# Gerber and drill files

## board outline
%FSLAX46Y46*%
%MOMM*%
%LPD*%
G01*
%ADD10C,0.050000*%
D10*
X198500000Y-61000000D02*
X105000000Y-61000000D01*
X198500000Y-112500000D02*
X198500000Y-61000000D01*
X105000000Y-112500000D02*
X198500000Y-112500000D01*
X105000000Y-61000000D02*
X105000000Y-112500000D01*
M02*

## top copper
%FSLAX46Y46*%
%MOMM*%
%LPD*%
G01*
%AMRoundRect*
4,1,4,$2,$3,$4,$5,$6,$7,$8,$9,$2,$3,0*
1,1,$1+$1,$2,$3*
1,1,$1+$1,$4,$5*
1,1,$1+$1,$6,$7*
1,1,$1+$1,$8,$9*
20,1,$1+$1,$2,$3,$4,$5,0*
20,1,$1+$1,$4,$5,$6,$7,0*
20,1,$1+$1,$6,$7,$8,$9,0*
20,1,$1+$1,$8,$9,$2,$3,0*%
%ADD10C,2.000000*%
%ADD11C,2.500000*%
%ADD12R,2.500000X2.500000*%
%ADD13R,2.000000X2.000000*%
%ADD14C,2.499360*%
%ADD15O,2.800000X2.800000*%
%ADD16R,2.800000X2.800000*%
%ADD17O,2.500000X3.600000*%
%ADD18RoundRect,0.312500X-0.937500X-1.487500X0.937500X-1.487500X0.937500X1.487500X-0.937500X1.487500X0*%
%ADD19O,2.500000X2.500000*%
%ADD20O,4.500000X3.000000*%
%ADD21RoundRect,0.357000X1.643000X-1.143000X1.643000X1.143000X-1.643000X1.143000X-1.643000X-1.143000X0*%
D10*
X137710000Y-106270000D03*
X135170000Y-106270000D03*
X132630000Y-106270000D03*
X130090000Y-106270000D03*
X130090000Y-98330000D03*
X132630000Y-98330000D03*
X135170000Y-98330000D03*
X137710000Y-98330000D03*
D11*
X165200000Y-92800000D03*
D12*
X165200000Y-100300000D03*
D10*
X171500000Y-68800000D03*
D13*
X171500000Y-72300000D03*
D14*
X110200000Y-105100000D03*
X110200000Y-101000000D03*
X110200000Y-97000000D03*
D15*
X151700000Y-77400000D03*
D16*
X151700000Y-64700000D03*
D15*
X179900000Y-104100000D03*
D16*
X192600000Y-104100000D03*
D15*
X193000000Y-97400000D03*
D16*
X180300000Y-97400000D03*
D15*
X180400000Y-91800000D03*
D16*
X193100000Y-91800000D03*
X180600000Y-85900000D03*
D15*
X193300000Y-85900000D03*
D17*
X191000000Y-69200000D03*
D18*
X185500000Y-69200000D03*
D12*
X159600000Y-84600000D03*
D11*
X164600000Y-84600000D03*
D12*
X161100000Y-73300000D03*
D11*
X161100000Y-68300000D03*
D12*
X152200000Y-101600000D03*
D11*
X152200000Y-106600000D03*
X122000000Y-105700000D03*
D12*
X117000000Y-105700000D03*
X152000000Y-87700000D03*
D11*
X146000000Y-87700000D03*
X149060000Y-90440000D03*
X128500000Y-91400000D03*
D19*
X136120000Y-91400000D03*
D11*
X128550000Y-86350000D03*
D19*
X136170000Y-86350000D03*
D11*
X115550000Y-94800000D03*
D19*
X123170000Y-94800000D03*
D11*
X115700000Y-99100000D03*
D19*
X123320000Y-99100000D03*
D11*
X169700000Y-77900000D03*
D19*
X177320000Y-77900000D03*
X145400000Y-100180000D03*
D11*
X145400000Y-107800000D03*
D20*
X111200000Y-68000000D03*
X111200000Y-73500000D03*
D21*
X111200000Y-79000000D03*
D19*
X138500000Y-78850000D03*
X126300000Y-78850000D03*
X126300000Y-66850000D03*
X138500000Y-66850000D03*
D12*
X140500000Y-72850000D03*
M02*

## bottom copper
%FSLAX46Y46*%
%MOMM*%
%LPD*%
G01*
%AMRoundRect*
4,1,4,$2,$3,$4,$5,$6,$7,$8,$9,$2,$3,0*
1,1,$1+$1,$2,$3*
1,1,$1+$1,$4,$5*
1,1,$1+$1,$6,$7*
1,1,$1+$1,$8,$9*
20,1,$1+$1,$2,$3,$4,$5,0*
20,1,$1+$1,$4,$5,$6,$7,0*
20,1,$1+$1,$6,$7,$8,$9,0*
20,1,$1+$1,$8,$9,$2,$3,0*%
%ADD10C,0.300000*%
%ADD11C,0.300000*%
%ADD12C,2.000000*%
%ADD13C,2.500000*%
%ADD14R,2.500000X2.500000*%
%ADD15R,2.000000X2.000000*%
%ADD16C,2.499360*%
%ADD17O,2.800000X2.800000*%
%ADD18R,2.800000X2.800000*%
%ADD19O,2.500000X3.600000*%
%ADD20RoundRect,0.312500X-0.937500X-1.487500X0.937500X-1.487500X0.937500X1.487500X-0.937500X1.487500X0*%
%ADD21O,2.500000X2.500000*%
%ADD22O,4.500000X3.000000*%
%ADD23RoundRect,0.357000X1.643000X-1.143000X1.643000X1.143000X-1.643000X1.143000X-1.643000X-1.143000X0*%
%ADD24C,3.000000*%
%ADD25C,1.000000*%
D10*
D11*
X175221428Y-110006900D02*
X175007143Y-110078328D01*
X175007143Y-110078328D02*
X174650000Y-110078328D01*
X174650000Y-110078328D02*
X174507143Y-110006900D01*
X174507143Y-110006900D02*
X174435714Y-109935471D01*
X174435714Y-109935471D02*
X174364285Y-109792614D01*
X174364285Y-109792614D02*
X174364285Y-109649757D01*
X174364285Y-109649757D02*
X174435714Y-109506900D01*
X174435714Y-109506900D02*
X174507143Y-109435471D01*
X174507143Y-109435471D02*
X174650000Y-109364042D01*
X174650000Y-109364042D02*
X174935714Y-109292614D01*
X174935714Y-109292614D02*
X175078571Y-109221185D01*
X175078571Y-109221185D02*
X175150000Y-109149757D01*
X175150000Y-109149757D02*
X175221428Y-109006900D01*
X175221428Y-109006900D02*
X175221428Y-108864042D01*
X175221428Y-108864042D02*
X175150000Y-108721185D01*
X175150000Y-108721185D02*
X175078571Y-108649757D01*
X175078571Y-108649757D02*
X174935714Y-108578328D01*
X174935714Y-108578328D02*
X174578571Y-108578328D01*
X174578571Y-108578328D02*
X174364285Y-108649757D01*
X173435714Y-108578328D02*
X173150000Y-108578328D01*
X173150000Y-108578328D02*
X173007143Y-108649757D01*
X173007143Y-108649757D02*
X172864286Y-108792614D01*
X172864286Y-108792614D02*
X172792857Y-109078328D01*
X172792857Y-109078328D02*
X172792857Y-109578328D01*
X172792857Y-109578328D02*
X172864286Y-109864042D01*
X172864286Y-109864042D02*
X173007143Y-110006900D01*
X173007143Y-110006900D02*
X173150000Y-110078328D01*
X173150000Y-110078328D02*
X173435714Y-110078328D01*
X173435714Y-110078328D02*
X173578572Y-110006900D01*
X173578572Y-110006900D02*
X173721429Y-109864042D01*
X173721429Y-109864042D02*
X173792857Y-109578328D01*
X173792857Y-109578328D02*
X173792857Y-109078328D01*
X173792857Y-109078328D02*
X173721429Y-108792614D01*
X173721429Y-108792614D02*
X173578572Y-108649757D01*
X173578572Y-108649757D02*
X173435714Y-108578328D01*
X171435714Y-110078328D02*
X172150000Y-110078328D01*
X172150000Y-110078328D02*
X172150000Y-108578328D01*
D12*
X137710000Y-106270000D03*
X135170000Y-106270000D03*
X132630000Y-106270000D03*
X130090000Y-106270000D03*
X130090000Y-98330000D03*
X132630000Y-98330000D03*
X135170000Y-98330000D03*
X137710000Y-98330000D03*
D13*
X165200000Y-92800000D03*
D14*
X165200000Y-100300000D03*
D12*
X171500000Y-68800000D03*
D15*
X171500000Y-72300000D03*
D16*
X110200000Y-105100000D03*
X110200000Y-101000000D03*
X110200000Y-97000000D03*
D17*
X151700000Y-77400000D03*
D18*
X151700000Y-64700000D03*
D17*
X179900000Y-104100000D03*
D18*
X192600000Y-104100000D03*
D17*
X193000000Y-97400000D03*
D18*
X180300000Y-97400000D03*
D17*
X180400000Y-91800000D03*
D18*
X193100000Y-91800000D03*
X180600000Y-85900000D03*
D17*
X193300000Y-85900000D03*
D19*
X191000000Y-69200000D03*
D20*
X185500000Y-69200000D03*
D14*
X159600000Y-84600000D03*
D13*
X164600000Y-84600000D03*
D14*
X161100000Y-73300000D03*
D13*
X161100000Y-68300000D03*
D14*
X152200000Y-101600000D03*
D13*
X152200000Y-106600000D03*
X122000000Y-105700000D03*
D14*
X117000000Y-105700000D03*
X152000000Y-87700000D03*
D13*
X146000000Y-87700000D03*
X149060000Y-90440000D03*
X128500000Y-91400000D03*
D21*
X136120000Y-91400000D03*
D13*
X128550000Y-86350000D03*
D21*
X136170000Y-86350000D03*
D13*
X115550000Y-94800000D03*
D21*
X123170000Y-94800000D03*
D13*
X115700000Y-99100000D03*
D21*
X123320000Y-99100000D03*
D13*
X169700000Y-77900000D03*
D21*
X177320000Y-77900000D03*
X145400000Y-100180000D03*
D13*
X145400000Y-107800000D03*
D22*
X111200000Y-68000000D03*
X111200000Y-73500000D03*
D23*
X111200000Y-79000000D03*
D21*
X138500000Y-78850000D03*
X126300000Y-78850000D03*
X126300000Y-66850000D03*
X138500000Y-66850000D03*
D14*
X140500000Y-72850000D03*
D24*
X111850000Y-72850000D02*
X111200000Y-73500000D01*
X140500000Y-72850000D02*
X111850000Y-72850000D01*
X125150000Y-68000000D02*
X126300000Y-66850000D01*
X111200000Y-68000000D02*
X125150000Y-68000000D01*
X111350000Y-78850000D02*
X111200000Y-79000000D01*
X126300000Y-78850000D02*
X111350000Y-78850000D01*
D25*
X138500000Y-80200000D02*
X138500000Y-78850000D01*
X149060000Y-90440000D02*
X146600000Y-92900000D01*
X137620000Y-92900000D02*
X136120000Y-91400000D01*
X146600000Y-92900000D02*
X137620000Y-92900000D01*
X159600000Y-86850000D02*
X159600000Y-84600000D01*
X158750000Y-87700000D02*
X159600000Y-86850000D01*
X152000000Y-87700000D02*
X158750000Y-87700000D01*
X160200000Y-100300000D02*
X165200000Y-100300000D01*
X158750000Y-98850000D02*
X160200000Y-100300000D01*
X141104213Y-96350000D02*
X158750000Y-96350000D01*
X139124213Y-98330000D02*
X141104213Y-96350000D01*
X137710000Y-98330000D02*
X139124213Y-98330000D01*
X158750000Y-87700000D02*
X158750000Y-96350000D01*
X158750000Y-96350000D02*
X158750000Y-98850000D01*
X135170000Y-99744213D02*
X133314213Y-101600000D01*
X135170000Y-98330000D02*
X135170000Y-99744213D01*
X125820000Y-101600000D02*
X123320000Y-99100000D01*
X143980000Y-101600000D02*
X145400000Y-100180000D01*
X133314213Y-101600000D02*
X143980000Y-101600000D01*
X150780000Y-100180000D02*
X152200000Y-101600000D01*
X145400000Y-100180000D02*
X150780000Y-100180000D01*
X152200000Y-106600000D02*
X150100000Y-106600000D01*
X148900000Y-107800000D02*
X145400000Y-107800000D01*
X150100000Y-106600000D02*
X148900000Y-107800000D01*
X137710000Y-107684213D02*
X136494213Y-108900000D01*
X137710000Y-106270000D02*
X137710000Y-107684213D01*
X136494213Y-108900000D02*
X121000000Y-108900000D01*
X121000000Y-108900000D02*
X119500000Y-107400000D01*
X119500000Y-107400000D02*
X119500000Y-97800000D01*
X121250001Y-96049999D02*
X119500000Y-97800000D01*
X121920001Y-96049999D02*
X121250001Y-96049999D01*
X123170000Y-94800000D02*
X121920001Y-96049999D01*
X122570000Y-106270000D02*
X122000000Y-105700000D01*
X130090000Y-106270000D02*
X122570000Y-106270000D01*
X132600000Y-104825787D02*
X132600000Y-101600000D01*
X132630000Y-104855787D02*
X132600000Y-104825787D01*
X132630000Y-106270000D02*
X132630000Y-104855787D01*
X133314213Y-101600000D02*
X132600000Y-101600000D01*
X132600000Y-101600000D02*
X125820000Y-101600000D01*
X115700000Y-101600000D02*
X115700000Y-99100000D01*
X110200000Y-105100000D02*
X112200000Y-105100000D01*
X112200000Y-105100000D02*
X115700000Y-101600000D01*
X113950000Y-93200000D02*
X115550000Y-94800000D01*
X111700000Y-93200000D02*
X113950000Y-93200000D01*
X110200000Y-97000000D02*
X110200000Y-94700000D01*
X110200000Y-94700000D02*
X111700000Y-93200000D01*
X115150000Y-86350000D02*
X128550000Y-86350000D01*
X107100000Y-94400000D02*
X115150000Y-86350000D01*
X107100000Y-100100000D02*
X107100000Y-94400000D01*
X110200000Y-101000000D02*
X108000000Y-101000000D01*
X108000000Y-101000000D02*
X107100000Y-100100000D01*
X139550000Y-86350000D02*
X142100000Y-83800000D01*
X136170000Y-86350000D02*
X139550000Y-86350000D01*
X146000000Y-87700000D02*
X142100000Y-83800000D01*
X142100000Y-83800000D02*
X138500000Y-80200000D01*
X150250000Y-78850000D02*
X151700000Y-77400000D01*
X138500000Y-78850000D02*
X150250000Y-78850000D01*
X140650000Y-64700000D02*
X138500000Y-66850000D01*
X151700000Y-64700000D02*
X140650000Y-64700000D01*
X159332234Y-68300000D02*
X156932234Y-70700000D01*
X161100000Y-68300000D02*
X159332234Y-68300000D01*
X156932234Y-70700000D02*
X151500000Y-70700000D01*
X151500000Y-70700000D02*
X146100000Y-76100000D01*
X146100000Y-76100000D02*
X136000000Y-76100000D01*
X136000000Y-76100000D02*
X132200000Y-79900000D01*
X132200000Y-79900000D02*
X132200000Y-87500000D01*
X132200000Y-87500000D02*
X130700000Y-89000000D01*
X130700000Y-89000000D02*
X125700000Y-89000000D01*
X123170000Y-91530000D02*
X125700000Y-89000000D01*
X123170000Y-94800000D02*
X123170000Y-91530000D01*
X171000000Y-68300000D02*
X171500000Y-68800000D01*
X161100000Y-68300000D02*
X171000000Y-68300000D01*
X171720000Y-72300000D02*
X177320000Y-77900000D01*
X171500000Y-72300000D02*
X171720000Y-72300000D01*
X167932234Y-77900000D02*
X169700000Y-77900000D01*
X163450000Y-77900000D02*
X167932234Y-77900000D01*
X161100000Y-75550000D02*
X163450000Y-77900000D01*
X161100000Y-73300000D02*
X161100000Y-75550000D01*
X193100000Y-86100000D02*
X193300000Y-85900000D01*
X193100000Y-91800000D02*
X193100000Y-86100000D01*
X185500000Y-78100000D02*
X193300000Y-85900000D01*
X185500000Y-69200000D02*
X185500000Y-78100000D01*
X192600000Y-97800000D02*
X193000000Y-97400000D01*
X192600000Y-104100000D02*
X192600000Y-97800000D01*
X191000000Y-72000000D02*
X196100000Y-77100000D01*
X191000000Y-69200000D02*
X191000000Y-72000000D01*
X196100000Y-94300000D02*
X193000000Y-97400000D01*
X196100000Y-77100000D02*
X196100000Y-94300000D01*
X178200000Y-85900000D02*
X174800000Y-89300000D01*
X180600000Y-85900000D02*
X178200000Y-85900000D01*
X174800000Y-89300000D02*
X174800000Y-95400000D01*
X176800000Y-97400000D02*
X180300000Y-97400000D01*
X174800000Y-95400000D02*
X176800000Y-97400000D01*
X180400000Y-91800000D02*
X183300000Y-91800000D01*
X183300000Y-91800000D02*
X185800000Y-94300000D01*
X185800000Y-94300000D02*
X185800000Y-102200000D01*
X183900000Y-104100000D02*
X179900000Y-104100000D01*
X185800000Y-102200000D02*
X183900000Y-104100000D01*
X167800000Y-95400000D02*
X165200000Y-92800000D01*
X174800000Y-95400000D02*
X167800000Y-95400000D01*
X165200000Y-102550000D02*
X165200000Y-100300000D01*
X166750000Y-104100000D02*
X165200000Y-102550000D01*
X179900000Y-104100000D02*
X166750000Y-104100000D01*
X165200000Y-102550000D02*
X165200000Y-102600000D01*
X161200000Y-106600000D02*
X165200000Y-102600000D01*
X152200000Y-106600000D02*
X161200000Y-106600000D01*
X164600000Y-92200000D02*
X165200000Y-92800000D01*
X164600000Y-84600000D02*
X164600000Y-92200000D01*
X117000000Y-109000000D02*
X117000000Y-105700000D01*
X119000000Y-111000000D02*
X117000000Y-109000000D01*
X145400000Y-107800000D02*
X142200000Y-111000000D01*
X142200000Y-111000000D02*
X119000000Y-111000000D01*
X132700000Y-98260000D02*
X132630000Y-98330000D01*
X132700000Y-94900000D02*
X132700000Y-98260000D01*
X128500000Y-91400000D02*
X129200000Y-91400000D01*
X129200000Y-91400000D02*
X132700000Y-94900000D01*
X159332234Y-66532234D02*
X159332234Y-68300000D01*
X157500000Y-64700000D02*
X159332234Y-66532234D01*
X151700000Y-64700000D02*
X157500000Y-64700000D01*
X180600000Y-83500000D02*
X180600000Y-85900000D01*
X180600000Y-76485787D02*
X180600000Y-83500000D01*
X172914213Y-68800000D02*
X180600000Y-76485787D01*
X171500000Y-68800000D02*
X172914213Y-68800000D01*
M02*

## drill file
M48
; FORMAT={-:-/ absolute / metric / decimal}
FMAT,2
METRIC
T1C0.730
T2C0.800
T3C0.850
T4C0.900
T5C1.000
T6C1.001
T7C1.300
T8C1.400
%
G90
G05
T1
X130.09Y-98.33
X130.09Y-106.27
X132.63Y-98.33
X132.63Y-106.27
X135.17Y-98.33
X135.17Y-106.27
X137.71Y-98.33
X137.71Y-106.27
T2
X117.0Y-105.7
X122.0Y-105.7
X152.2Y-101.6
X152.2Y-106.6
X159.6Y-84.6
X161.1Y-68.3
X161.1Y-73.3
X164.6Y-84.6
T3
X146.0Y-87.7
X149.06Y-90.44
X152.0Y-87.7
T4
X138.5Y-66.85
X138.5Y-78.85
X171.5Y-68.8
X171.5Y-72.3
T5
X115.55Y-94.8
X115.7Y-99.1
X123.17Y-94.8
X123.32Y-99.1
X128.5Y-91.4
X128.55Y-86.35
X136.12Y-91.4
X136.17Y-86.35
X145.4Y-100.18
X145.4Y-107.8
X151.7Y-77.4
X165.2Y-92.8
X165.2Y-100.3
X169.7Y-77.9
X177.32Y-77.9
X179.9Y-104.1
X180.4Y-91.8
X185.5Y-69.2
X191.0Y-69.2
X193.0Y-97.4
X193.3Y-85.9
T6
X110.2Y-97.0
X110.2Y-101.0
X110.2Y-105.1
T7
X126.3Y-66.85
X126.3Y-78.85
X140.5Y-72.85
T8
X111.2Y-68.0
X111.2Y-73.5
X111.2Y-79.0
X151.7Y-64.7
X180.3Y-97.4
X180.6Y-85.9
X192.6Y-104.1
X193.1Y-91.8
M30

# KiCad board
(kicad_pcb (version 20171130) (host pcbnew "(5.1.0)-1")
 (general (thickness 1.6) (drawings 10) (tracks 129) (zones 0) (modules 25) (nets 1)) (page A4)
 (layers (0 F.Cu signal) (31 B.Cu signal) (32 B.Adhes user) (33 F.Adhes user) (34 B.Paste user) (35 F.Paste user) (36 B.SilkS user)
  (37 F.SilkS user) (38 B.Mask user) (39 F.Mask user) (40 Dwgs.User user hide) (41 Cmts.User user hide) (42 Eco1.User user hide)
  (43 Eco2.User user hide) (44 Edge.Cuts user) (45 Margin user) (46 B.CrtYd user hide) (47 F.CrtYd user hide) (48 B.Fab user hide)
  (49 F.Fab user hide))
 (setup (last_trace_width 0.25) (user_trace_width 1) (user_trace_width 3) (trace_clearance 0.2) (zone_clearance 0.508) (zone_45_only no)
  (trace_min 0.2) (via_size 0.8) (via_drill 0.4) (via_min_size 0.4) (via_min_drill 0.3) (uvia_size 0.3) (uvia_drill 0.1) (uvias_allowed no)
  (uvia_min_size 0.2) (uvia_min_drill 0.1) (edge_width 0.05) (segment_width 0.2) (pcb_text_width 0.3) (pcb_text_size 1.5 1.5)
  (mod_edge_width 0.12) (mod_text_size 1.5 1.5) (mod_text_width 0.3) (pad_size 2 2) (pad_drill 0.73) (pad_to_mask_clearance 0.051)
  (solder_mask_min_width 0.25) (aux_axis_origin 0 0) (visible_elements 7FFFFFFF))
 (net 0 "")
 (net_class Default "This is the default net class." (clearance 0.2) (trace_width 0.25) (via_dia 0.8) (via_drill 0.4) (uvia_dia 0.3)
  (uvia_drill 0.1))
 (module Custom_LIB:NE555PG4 (layer F.Cu) (at 133.9 102.3 270)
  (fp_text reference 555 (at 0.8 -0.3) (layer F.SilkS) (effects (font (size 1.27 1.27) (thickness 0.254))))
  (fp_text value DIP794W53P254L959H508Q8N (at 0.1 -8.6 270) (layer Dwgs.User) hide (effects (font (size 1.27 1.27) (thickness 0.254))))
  (pad 8 thru_hole circle (at 3.97 -3.81 270) (size 2 2) (drill 0.73) (layers *.Cu *.Mask))
  (pad 7 thru_hole circle (at 3.97 -1.27 270) (size 2 2) (drill 0.73) (layers *.Cu *.Mask))
  (pad 6 thru_hole circle (at 3.97 1.27 270) (size 2 2) (drill 0.73) (layers *.Cu *.Mask))
  (pad 5 thru_hole circle (at 3.97 3.81 270) (size 2 2) (drill 0.73) (layers *.Cu *.Mask))
  (pad 4 thru_hole circle (at -3.97 3.81 270) (size 2 2) (drill 0.73) (layers *.Cu *.Mask))
  (pad 3 thru_hole circle (at -3.97 1.27 270) (size 2 2) (drill 0.73) (layers *.Cu *.Mask))
  (pad 2 thru_hole circle (at -3.97 -1.27 270) (size 2 2) (drill 0.73) (layers *.Cu *.Mask))
  (pad 1 thru_hole circle (at -3.97 -3.81 270) (size 2 2) (drill 0.73) (layers *.Cu *.Mask)))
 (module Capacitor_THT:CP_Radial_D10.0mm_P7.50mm (layer F.Cu) (at 165.2 100.3 90)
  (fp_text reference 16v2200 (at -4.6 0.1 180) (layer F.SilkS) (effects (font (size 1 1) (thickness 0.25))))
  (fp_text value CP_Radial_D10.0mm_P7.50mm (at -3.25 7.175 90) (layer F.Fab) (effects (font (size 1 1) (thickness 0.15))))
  (pad 2 thru_hole circle (at 7.5 0 90) (size 2.5 2.5) (drill 1) (layers *.Cu *.Mask))
  (pad 1 thru_hole rect (at 0 0 90) (size 2.5 2.5) (drill 1) (layers *.Cu *.Mask)))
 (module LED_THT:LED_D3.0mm (layer F.Cu) (at 171.5 71.8 90)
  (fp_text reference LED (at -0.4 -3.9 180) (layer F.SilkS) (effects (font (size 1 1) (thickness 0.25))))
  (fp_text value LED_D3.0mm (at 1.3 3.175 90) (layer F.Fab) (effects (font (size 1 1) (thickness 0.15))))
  (pad 2 thru_hole circle (at 3 0 180) (size 2 2) (drill 0.9) (layers *.Cu *.Mask))
  (pad 1 thru_hole rect (at -0.5 0 90) (size 2 2) (drill 0.9) (layers *.Cu *.Mask)))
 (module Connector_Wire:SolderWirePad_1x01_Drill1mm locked (layer F.Cu) (at 110.2 105.1)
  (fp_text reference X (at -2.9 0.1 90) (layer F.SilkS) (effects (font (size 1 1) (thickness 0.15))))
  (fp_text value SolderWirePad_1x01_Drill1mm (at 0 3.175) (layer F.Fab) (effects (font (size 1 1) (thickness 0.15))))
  (pad 1 thru_hole circle (at 0 0) (size 2.49936 2.49936) (drill 1.00076) (layers *.Cu *.Mask)))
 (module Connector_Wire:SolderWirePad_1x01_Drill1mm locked (layer F.Cu) (at 110.2 101)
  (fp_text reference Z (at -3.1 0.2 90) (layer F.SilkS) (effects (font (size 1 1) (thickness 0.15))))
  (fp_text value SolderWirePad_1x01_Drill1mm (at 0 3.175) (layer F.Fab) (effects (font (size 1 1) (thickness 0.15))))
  (pad 1 thru_hole circle (at 0 0) (size 2.49936 2.49936) (drill 1.00076) (layers *.Cu *.Mask)))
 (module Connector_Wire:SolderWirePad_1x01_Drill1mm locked (layer F.Cu) (at 110.5 97)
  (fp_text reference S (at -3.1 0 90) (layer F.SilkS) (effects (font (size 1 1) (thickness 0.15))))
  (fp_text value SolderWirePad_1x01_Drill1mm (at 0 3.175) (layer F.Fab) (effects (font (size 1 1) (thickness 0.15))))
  (pad 1 thru_hole circle (at -0.3 0) (size 2.49936 2.49936) (drill 1.00076) (layers *.Cu *.Mask)))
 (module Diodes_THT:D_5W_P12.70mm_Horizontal (layer F.Cu) (at 151.7 64.7 270)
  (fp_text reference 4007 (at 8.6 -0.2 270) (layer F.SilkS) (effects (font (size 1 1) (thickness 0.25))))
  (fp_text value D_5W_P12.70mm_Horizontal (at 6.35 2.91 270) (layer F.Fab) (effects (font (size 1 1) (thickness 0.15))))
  (pad 2 thru_hole oval (at 12.7 0 270) (size 2.8 2.8) (drill 1) (layers *.Cu *.Mask))
  (pad 1 thru_hole rect (at 0 0 270) (size 2.8 2.8) (drill 1.4) (layers *.Cu *.Mask)))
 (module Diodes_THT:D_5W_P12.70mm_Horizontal (layer F.Cu) (at 192.6 104.1 180)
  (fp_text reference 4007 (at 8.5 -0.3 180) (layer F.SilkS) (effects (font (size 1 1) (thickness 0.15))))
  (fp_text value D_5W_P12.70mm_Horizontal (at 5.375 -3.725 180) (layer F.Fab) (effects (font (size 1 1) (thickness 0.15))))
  (pad 2 thru_hole oval (at 12.7 0 180) (size 2.8 2.8) (drill 1) (layers *.Cu *.Mask))
  (pad 1 thru_hole rect (at 0 0 180) (size 2.8 2.8) (drill 1.4) (layers *.Cu *.Mask)))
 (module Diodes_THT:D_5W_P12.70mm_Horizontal (layer F.Cu) (at 180.3 97.4)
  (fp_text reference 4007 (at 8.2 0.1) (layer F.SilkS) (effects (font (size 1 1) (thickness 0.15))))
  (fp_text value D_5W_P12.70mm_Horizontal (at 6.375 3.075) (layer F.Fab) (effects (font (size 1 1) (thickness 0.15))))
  (pad 2 thru_hole oval (at 12.7 0) (size 2.8 2.8) (drill 1) (layers *.Cu *.Mask))
  (pad 1 thru_hole rect (at 0 0) (size 2.8 2.8) (drill 1.4) (layers *.Cu *.Mask)))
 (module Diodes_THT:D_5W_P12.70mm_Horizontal (layer F.Cu) (at 193.1 91.8 180)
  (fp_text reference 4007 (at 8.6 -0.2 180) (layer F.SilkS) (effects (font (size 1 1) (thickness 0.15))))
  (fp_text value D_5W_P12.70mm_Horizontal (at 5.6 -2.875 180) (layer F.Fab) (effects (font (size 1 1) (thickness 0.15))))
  (pad 2 thru_hole oval (at 12.7 0 180) (size 2.8 2.8) (drill 1) (layers *.Cu *.Mask))
  (pad 1 thru_hole rect (at 0 0 180) (size 2.8 2.8) (drill 1.4) (layers *.Cu *.Mask)))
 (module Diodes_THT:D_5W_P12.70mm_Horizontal (layer F.Cu) (at 180.6 85.9)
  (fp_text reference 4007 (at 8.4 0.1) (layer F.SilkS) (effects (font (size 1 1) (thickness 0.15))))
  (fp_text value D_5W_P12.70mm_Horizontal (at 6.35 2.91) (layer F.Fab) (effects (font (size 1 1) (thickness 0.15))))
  (pad 1 thru_hole rect (at 0 0) (size 2.8 2.8) (drill 1.4) (layers *.Cu *.Mask))
  (pad 2 thru_hole oval (at 12.7 0) (size 2.8 2.8) (drill 1) (layers *.Cu *.Mask)))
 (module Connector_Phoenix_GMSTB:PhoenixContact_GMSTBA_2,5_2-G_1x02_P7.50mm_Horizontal (layer F.Cu) (at 184.5 66.2)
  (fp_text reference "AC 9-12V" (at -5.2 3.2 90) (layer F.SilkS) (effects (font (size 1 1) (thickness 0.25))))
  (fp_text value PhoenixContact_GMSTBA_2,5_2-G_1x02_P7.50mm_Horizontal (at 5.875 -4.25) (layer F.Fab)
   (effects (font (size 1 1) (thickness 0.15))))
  (pad 2 thru_hole oval (at 6.5 3) (size 2.5 3.6) (drill 1) (layers *.Cu *.Mask))
  (pad 1 thru_hole roundrect (at 1 3) (size 2.5 3.6) (drill 1) (layers *.Cu *.Mask) (roundrect_rratio 0.125)))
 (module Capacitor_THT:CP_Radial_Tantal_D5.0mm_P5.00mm (layer F.Cu) (at 159.6 84.6)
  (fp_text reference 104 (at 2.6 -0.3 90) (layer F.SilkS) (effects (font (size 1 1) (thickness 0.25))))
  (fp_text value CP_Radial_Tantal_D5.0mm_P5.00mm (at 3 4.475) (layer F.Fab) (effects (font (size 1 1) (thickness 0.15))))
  (pad 1 thru_hole rect (at 0 0) (size 2.5 2.5) (drill 0.8) (layers *.Cu *.Mask))
  (pad 2 thru_hole circle (at 5 0) (size 2.5 2.5) (drill 0.8) (layers *.Cu *.Mask)))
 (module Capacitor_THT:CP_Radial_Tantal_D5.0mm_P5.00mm (layer F.Cu) (at 161.1 73.3 90)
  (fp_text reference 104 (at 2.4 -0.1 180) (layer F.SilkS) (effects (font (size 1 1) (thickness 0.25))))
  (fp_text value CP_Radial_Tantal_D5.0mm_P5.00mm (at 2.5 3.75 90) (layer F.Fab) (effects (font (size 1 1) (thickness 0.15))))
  (pad 1 thru_hole rect (at 0 0 90) (size 2.5 2.5) (drill 0.8) (layers *.Cu *.Mask))
  (pad 2 thru_hole circle (at 5 0 90) (size 2.5 2.5) (drill 0.8) (layers *.Cu *.Mask)))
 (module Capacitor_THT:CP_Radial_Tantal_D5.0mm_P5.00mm (layer F.Cu) (at 152.2 101.6 270)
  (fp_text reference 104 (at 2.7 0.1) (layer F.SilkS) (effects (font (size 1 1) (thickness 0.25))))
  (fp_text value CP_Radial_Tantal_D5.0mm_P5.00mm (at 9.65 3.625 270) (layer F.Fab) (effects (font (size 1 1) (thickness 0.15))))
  (pad 1 thru_hole rect (at 0 0 270) (size 2.5 2.5) (drill 0.8) (layers *.Cu *.Mask))
  (pad 2 thru_hole circle (at 5 0 270) (size 2.5 2.5) (drill 0.8) (layers *.Cu *.Mask)))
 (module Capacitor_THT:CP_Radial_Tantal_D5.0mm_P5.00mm (layer F.Cu) (at 117 105.7)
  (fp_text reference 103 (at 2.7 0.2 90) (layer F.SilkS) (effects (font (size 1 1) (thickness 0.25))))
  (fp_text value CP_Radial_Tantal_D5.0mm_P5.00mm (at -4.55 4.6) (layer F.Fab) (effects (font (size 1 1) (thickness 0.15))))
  (pad 2 thru_hole circle (at 5 0) (size 2.5 2.5) (drill 0.8) (layers *.Cu *.Mask))
  (pad 1 thru_hole rect (at 0 0) (size 2.5 2.5) (drill 0.8) (layers *.Cu *.Mask)))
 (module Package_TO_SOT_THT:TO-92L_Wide (layer F.Cu) (at 151.6 87.9 180)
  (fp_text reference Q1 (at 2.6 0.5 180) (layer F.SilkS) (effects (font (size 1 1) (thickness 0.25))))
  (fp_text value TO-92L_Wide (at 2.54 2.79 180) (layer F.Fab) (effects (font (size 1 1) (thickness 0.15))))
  (pad 1 thru_hole rect (at -0.4 0.2 270) (size 2.5 2.5) (drill 0.85) (layers *.Cu *.Mask))
  (pad 3 thru_hole circle (at 5.6 0.2 270) (size 2.5 2.5) (drill 0.85) (layers *.Cu *.Mask))
  (pad 2 thru_hole circle (at 2.54 -2.54 270) (size 2.5 2.5) (drill 0.85) (layers *.Cu *.Mask)))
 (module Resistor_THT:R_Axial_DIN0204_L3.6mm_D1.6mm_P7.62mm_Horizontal (layer F.Cu) (at 128.5 91.4)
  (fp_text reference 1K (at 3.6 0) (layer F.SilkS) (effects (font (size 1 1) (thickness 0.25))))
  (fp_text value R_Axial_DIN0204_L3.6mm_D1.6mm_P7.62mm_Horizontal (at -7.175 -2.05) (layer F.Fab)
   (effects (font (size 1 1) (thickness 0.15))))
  (pad 1 thru_hole circle (at 0 0) (size 2.5 2.5) (drill 1) (layers *.Cu *.Mask))
  (pad 2 thru_hole oval (at 7.62 0 90) (size 2.5 2.5) (drill 1) (layers *.Cu *.Mask)))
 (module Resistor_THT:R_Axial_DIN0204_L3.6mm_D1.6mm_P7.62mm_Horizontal (layer F.Cu) (at 128.55 86.35)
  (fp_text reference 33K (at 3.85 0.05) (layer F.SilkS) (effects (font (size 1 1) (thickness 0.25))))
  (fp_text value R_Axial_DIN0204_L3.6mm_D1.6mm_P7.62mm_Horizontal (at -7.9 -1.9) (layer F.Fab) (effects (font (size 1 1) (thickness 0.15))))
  (pad 1 thru_hole circle (at 0 0) (size 2.5 2.5) (drill 1) (layers *.Cu *.Mask))
  (pad 2 thru_hole oval (at 7.62 0 90) (size 2.5 2.5) (drill 1) (layers *.Cu *.Mask)))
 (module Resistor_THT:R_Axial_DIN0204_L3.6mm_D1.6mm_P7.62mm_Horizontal (layer F.Cu) (at 115.55 94.8)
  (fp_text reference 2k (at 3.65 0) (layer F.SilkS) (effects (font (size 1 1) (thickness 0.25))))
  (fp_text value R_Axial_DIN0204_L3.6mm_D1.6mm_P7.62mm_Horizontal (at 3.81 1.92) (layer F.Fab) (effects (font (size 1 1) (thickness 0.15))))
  (pad 1 thru_hole circle (at 0 0) (size 2.5 2.5) (drill 1) (layers *.Cu *.Mask))
  (pad 2 thru_hole oval (at 7.62 0 90) (size 2.5 2.5) (drill 1) (layers *.Cu *.Mask)))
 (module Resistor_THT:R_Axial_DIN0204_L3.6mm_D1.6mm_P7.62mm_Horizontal (layer F.Cu) (at 115.7 99.1)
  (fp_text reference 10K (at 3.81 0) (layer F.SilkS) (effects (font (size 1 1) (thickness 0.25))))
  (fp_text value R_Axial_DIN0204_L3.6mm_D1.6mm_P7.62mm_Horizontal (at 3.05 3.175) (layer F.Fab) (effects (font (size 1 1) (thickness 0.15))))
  (pad 1 thru_hole circle (at 0 0) (size 2.5 2.5) (drill 1) (layers *.Cu *.Mask))
  (pad 2 thru_hole oval (at 7.62 0 90) (size 2.5 2.5) (drill 1) (layers *.Cu *.Mask)))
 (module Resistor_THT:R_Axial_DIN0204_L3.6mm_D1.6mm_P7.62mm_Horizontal (layer F.Cu) (at 169.7 77.9)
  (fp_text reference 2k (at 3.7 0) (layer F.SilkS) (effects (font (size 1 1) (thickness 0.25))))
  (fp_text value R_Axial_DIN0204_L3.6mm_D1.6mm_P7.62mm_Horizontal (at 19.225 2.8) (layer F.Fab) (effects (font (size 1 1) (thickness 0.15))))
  (pad 1 thru_hole circle (at 0 0) (size 2.5 2.5) (drill 1) (layers *.Cu *.Mask))
  (pad 2 thru_hole oval (at 7.62 0 90) (size 2.5 2.5) (drill 1) (layers *.Cu *.Mask)))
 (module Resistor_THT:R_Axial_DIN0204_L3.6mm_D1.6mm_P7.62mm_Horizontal (layer F.Cu) (at 145.4 107.8 90)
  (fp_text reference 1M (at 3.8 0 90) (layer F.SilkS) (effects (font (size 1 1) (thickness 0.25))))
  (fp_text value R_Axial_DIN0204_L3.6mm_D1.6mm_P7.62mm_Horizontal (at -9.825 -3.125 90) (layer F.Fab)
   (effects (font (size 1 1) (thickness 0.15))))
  (pad 2 thru_hole oval (at 7.62 0 180) (size 2.5 2.5) (drill 1) (layers *.Cu *.Mask))
  (pad 1 thru_hole circle (at 0 0 90) (size 2.5 2.5) (drill 1) (layers *.Cu *.Mask)))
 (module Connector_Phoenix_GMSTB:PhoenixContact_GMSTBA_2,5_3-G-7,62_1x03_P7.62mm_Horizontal (layer F.Cu) (at 108.5 81 90)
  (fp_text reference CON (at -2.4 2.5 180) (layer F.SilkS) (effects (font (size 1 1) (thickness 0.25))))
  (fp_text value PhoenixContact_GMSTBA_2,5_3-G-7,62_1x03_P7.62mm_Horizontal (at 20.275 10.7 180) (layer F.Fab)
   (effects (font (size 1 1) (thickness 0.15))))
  (pad 3 thru_hole oval (at 13 2.7 90) (size 3 4.5) (drill 1.4) (layers *.Cu *.Mask))
  (pad 2 thru_hole oval (at 7.5 2.7 90) (size 3 4.5) (drill 1.4) (layers *.Cu *.Mask))
  (pad 1 thru_hole roundrect (at 2 2.7 90) (size 3 4) (drill 1.4) (layers *.Cu *.Mask) (roundrect_rratio 0.119)))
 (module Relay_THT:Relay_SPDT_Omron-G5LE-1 (layer F.Cu) (at 140.5 72.85 270)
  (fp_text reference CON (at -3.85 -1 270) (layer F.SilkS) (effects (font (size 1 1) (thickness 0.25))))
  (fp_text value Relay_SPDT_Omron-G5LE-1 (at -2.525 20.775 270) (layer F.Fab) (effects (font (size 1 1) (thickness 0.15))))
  (pad 5 thru_hole oval (at 6 2 270) (size 2.5 2.5) (drill 0.9) (layers *.Cu *.Mask))
  (pad 4 thru_hole oval (at 6 14.2 270) (size 2.5 2.5) (drill 1.3) (layers *.Cu *.Mask))
  (pad 3 thru_hole oval (at -6 14.2 270) (size 2.5 2.5) (drill 1.3) (layers *.Cu *.Mask))
  (pad 2 thru_hole oval (at -6 2 270) (size 2.5 2.5) (drill 0.9) (layers *.Cu *.Mask))
  (pad 1 thru_hole rect (at 0 0 270) (size 2.5 2.5) (drill 1.3) (layers *.Cu *.Mask)))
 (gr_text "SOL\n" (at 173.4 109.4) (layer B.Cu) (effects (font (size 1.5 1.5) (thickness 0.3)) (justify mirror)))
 (gr_line (start 198.5 61) (end 105 61) (layer Edge.Cuts) (width 0.05))
 (gr_line (start 198.5 112.5) (end 198.5 61) (layer Edge.Cuts) (width 0.05))
 (gr_line (start 105 112.5) (end 198.5 112.5) (layer Edge.Cuts) (width 0.05))
 (gr_line (start 105 61) (end 105 112.5) (layer Edge.Cuts) (width 0.05))
 (segment (start 111.85 72.85) (end 111.2 73.5) (width 3) (layer B.Cu) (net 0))
 (segment (start 140.5 72.85) (end 111.85 72.85) (width 3) (layer B.Cu) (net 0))
 (segment (start 125.15 68) (end 126.3 66.85) (width 3) (layer B.Cu) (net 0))
 (segment (start 111.2 68) (end 125.15 68) (width 3) (layer B.Cu) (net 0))
 (segment (start 111.35 78.85) (end 111.2 79) (width 3) (layer B.Cu) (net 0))
 (segment (start 126.3 78.85) (end 111.35 78.85) (width 3) (layer B.Cu) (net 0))
 (segment (start 138.5 80.2) (end 138.5 78.85) (width 1) (layer B.Cu) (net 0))
 (segment (start 149.06 90.44) (end 146.6 92.9) (width 1) (layer B.Cu) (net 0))
 (segment (start 137.62 92.9) (end 136.12 91.4) (width 1) (layer B.Cu) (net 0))
 (segment (start 146.6 92.9) (end 137.62 92.9) (width 1) (layer B.Cu) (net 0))
 (segment (start 159.6 86.85) (end 159.6 84.6) (width 1) (layer B.Cu) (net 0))
 (segment (start 158.75 87.7) (end 159.6 86.85) (width 1) (layer B.Cu) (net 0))
 (segment (start 152 87.7) (end 158.75 87.7) (width 1) (layer B.Cu) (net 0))
 (segment (start 160.2 100.3) (end 165.2 100.3) (width 1) (layer B.Cu) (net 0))
 (segment (start 158.75 98.85) (end 160.2 100.3) (width 1) (layer B.Cu) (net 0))
 (segment (start 141.104213 96.35) (end 158.75 96.35) (width 1) (layer B.Cu) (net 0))
 (segment (start 139.124213 98.33) (end 141.104213 96.35) (width 1) (layer B.Cu) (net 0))
 (segment (start 137.71 98.33) (end 139.124213 98.33) (width 1) (layer B.Cu) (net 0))
 (segment (start 158.75 87.7) (end 158.75 96.35) (width 1) (layer B.Cu) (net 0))
 (segment (start 158.75 96.35) (end 158.75 98.85) (width 1) (layer B.Cu) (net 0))
 (segment (start 135.17 99.744213) (end 133.314213 101.6) (width 1) (layer B.Cu) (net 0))
 (segment (start 135.17 98.33) (end 135.17 99.744213) (width 1) (layer B.Cu) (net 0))
 (segment (start 125.82 101.6) (end 123.32 99.1) (width 1) (layer B.Cu) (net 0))
 (segment (start 143.98 101.6) (end 145.4 100.18) (width 1) (layer B.Cu) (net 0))
 (segment (start 133.314213 101.6) (end 143.98 101.6) (width 1) (layer B.Cu) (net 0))
 (segment (start 150.78 100.18) (end 152.2 101.6) (width 1) (layer B.Cu) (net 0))
 (segment (start 145.4 100.18) (end 150.78 100.18) (width 1) (layer B.Cu) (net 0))
 (segment (start 152.2 106.6) (end 150.1 106.6) (width 1) (layer B.Cu) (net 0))
 (segment (start 148.9 107.8) (end 145.4 107.8) (width 1) (layer B.Cu) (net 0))
 (segment (start 150.1 106.6) (end 148.9 107.8) (width 1) (layer B.Cu) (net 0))
 (segment (start 137.71 107.684213) (end 136.494213 108.9) (width 1) (layer B.Cu) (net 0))
 (segment (start 137.71 106.27) (end 137.71 107.684213) (width 1) (layer B.Cu) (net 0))
 (segment (start 136.494213 108.9) (end 121 108.9) (width 1) (layer B.Cu) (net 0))
 (segment (start 121 108.9) (end 119.5 107.4) (width 1) (layer B.Cu) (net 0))
 (segment (start 119.5 107.4) (end 119.5 97.8) (width 1) (layer B.Cu) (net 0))
 (segment (start 121.250001 96.049999) (end 119.5 97.8) (width 1) (layer B.Cu) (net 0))
 (segment (start 121.920001 96.049999) (end 121.250001 96.049999) (width 1) (layer B.Cu) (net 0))
 (segment (start 123.17 94.8) (end 121.920001 96.049999) (width 1) (layer B.Cu) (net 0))
 (segment (start 122.57 106.27) (end 122 105.7) (width 1) (layer B.Cu) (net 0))
 (segment (start 130.09 106.27) (end 122.57 106.27) (width 1) (layer B.Cu) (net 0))
 (segment (start 132.6 104.825787) (end 132.6 101.6) (width 1) (layer B.Cu) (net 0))
 (segment (start 132.63 104.855787) (end 132.6 104.825787) (width 1) (layer B.Cu) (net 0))
 (segment (start 132.63 106.27) (end 132.63 104.855787) (width 1) (layer B.Cu) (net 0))
 (segment (start 133.314213 101.6) (end 132.6 101.6) (width 1) (layer B.Cu) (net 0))
 (segment (start 132.6 101.6) (end 125.82 101.6) (width 1) (layer B.Cu) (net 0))
 (segment (start 115.7 101.6) (end 115.7 99.1) (width 1) (layer B.Cu) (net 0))
 (segment (start 110.2 105.1) (end 112.2 105.1) (width 1) (layer B.Cu) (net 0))
 (segment (start 112.2 105.1) (end 115.7 101.6) (width 1) (layer B.Cu) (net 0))
 (segment (start 113.95 93.2) (end 115.55 94.8) (width 1) (layer B.Cu) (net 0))
 (segment (start 111.7 93.2) (end 113.95 93.2) (width 1) (layer B.Cu) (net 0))
 (segment (start 110.2 97) (end 110.2 94.7) (width 1) (layer B.Cu) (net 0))
 (segment (start 110.2 94.7) (end 111.7 93.2) (width 1) (layer B.Cu) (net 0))
 (segment (start 115.15 86.35) (end 128.55 86.35) (width 1) (layer B.Cu) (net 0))
 (segment (start 107.1 94.4) (end 115.15 86.35) (width 1) (layer B.Cu) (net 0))
 (segment (start 107.1 100.1) (end 107.1 94.4) (width 1) (layer B.Cu) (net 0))
 (segment (start 110.2 101) (end 108 101) (width 1) (layer B.Cu) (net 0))
 (segment (start 108 101) (end 107.1 100.1) (width 1) (layer B.Cu) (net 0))
 (segment (start 139.55 86.35) (end 142.1 83.8) (width 1) (layer B.Cu) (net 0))
 (segment (start 136.17 86.35) (end 139.55 86.35) (width 1) (layer B.Cu) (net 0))
 (segment (start 146 87.7) (end 142.1 83.8) (width 1) (layer B.Cu) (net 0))
 (segment (start 142.1 83.8) (end 138.5 80.2) (width 1) (layer B.Cu) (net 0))
 (segment (start 150.25 78.85) (end 151.7 77.4) (width 1) (layer B.Cu) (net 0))
 (segment (start 138.5 78.85) (end 150.25 78.85) (width 1) (layer B.Cu) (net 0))
 (segment (start 140.65 64.7) (end 138.5 66.85) (width 1) (layer B.Cu) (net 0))
 (segment (start 151.7 64.7) (end 140.65 64.7) (width 1) (layer B.Cu) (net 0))
 (segment (start 159.332234 68.3) (end 156.932234 70.7) (width 1) (layer B.Cu) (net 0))
 (segment (start 161.1 68.3) (end 159.332234 68.3) (width 1) (layer B.Cu) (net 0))
 (segment (start 156.932234 70.7) (end 151.5 70.7) (width 1) (layer B.Cu) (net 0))
 (segment (start 151.5 70.7) (end 146.1 76.1) (width 1) (layer B.Cu) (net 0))
 (segment (start 146.1 76.1) (end 136 76.1) (width 1) (layer B.Cu) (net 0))
 (segment (start 136 76.1) (end 132.2 79.9) (width 1) (layer B.Cu) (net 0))
 (segment (start 132.2 79.9) (end 132.2 87.5) (width 1) (layer B.Cu) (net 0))
 (segment (start 132.2 87.5) (end 130.7 89) (width 1) (layer B.Cu) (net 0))
 (segment (start 130.7 89) (end 125.7 89) (width 1) (layer B.Cu) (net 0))
 (segment (start 123.17 91.53) (end 125.7 89) (width 1) (layer B.Cu) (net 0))
 (segment (start 123.17 94.8) (end 123.17 91.53) (width 1) (layer B.Cu) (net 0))
 (segment (start 171 68.3) (end 171.5 68.8) (width 1) (layer B.Cu) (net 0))
 (segment (start 161.1 68.3) (end 171 68.3) (width 1) (layer B.Cu) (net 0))
 (segment (start 171.72 72.3) (end 177.32 77.9) (width 1) (layer B.Cu) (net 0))
 (segment (start 171.5 72.3) (end 171.72 72.3) (width 1) (layer B.Cu) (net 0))
 (segment (start 167.932234 77.9) (end 169.7 77.9) (width 1) (layer B.Cu) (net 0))
 (segment (start 163.45 77.9) (end 167.932234 77.9) (width 1) (layer B.Cu) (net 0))
 (segment (start 161.1 75.55) (end 163.45 77.9) (width 1) (layer B.Cu) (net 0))
 (segment (start 161.1 73.3) (end 161.1 75.55) (width 1) (layer B.Cu) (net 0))
 (segment (start 193.1 86.1) (end 193.3 85.9) (width 1) (layer B.Cu) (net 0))
 (segment (start 193.1 91.8) (end 193.1 86.1) (width 1) (layer B.Cu) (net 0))
 (segment (start 185.5 78.1) (end 193.3 85.9) (width 1) (layer B.Cu) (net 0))
 (segment (start 185.5 69.2) (end 185.5 78.1) (width 1) (layer B.Cu) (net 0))
 (segment (start 192.6 97.8) (end 193 97.4) (width 1) (layer B.Cu) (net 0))
 (segment (start 192.6 104.1) (end 192.6 97.8) (width 1) (layer B.Cu) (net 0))
 (segment (start 191 72) (end 196.1 77.1) (width 1) (layer B.Cu) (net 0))
 (segment (start 191 69.2) (end 191 72) (width 1) (layer B.Cu) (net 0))
 (segment (start 196.1 94.3) (end 193 97.4) (width 1) (layer B.Cu) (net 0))
 (segment (start 196.1 77.1) (end 196.1 94.3) (width 1) (layer B.Cu) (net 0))
 (segment (start 178.2 85.9) (end 174.8 89.3) (width 1) (layer B.Cu) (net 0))
 (segment (start 180.6 85.9) (end 178.2 85.9) (width 1) (layer B.Cu) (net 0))
 (segment (start 174.8 89.3) (end 174.8 95.4) (width 1) (layer B.Cu) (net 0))
 (segment (start 176.8 97.4) (end 180.3 97.4) (width 1) (layer B.Cu) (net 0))
 (segment (start 174.8 95.4) (end 176.8 97.4) (width 1) (layer B.Cu) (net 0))
 (segment (start 180.4 91.8) (end 183.3 91.8) (width 1) (layer B.Cu) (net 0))
 (segment (start 183.3 91.8) (end 185.8 94.3) (width 1) (layer B.Cu) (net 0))
 (segment (start 185.8 94.3) (end 185.8 102.2) (width 1) (layer B.Cu) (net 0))
 (segment (start 183.9 104.1) (end 179.9 104.1) (width 1) (layer B.Cu) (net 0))
 (segment (start 185.8 102.2) (end 183.9 104.1) (width 1) (layer B.Cu) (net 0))
 (segment (start 167.8 95.4) (end 165.2 92.8) (width 1) (layer B.Cu) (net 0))
 (segment (start 174.8 95.4) (end 167.8 95.4) (width 1) (layer B.Cu) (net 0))
 (segment (start 165.2 102.55) (end 165.2 100.3) (width 1) (layer B.Cu) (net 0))
 (segment (start 166.75 104.1) (end 165.2 102.55) (width 1) (layer B.Cu) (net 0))
 (segment (start 179.9 104.1) (end 166.75 104.1) (width 1) (layer B.Cu) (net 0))
 (segment (start 165.2 102.55) (end 165.2 102.6) (width 1) (layer B.Cu) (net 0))
 (segment (start 161.2 106.6) (end 165.2 102.6) (width 1) (layer B.Cu) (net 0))
 (segment (start 152.2 106.6) (end 161.2 106.6) (width 1) (layer B.Cu) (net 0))
 (segment (start 164.6 92.2) (end 165.2 92.8) (width 1) (layer B.Cu) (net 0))
 (segment (start 164.6 84.6) (end 164.6 92.2) (width 1) (layer B.Cu) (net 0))
 (segment (start 117 109) (end 117 105.7) (width 1) (layer B.Cu) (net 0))
 (segment (start 119 111) (end 117 109) (width 1) (layer B.Cu) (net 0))
 (segment (start 145.4 107.8) (end 142.2 111) (width 1) (layer B.Cu) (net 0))
 (segment (start 142.2 111) (end 119 111) (width 1) (layer B.Cu) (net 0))
 (segment (start 132.7 98.26) (end 132.63 98.33) (width 1) (layer B.Cu) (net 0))
 (segment (start 132.7 94.9) (end 132.7 98.26) (width 1) (layer B.Cu) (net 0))
 (segment (start 128.5 91.4) (end 129.2 91.4) (width 1) (layer B.Cu) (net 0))
 (segment (start 129.2 91.4) (end 132.7 94.9) (width 1) (layer B.Cu) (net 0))
 (segment (start 159.332234 66.532234) (end 159.332234 68.3) (width 1) (layer B.Cu) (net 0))
 (segment (start 157.5 64.7) (end 159.332234 66.532234) (width 1) (layer B.Cu) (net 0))
 (segment (start 151.7 64.7) (end 157.5 64.7) (width 1) (layer B.Cu) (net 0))
 (segment (start 180.6 83.5) (end 180.6 85.9) (width 1) (layer B.Cu) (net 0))
 (segment (start 180.6 76.485787) (end 180.6 83.5) (width 1) (layer B.Cu) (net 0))
 (segment (start 172.914213 68.8) (end 180.6 76.485787) (width 1) (layer B.Cu) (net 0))
 (segment (start 171.5 68.8) (end 172.914213 68.8) (width 1) (layer B.Cu) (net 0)))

